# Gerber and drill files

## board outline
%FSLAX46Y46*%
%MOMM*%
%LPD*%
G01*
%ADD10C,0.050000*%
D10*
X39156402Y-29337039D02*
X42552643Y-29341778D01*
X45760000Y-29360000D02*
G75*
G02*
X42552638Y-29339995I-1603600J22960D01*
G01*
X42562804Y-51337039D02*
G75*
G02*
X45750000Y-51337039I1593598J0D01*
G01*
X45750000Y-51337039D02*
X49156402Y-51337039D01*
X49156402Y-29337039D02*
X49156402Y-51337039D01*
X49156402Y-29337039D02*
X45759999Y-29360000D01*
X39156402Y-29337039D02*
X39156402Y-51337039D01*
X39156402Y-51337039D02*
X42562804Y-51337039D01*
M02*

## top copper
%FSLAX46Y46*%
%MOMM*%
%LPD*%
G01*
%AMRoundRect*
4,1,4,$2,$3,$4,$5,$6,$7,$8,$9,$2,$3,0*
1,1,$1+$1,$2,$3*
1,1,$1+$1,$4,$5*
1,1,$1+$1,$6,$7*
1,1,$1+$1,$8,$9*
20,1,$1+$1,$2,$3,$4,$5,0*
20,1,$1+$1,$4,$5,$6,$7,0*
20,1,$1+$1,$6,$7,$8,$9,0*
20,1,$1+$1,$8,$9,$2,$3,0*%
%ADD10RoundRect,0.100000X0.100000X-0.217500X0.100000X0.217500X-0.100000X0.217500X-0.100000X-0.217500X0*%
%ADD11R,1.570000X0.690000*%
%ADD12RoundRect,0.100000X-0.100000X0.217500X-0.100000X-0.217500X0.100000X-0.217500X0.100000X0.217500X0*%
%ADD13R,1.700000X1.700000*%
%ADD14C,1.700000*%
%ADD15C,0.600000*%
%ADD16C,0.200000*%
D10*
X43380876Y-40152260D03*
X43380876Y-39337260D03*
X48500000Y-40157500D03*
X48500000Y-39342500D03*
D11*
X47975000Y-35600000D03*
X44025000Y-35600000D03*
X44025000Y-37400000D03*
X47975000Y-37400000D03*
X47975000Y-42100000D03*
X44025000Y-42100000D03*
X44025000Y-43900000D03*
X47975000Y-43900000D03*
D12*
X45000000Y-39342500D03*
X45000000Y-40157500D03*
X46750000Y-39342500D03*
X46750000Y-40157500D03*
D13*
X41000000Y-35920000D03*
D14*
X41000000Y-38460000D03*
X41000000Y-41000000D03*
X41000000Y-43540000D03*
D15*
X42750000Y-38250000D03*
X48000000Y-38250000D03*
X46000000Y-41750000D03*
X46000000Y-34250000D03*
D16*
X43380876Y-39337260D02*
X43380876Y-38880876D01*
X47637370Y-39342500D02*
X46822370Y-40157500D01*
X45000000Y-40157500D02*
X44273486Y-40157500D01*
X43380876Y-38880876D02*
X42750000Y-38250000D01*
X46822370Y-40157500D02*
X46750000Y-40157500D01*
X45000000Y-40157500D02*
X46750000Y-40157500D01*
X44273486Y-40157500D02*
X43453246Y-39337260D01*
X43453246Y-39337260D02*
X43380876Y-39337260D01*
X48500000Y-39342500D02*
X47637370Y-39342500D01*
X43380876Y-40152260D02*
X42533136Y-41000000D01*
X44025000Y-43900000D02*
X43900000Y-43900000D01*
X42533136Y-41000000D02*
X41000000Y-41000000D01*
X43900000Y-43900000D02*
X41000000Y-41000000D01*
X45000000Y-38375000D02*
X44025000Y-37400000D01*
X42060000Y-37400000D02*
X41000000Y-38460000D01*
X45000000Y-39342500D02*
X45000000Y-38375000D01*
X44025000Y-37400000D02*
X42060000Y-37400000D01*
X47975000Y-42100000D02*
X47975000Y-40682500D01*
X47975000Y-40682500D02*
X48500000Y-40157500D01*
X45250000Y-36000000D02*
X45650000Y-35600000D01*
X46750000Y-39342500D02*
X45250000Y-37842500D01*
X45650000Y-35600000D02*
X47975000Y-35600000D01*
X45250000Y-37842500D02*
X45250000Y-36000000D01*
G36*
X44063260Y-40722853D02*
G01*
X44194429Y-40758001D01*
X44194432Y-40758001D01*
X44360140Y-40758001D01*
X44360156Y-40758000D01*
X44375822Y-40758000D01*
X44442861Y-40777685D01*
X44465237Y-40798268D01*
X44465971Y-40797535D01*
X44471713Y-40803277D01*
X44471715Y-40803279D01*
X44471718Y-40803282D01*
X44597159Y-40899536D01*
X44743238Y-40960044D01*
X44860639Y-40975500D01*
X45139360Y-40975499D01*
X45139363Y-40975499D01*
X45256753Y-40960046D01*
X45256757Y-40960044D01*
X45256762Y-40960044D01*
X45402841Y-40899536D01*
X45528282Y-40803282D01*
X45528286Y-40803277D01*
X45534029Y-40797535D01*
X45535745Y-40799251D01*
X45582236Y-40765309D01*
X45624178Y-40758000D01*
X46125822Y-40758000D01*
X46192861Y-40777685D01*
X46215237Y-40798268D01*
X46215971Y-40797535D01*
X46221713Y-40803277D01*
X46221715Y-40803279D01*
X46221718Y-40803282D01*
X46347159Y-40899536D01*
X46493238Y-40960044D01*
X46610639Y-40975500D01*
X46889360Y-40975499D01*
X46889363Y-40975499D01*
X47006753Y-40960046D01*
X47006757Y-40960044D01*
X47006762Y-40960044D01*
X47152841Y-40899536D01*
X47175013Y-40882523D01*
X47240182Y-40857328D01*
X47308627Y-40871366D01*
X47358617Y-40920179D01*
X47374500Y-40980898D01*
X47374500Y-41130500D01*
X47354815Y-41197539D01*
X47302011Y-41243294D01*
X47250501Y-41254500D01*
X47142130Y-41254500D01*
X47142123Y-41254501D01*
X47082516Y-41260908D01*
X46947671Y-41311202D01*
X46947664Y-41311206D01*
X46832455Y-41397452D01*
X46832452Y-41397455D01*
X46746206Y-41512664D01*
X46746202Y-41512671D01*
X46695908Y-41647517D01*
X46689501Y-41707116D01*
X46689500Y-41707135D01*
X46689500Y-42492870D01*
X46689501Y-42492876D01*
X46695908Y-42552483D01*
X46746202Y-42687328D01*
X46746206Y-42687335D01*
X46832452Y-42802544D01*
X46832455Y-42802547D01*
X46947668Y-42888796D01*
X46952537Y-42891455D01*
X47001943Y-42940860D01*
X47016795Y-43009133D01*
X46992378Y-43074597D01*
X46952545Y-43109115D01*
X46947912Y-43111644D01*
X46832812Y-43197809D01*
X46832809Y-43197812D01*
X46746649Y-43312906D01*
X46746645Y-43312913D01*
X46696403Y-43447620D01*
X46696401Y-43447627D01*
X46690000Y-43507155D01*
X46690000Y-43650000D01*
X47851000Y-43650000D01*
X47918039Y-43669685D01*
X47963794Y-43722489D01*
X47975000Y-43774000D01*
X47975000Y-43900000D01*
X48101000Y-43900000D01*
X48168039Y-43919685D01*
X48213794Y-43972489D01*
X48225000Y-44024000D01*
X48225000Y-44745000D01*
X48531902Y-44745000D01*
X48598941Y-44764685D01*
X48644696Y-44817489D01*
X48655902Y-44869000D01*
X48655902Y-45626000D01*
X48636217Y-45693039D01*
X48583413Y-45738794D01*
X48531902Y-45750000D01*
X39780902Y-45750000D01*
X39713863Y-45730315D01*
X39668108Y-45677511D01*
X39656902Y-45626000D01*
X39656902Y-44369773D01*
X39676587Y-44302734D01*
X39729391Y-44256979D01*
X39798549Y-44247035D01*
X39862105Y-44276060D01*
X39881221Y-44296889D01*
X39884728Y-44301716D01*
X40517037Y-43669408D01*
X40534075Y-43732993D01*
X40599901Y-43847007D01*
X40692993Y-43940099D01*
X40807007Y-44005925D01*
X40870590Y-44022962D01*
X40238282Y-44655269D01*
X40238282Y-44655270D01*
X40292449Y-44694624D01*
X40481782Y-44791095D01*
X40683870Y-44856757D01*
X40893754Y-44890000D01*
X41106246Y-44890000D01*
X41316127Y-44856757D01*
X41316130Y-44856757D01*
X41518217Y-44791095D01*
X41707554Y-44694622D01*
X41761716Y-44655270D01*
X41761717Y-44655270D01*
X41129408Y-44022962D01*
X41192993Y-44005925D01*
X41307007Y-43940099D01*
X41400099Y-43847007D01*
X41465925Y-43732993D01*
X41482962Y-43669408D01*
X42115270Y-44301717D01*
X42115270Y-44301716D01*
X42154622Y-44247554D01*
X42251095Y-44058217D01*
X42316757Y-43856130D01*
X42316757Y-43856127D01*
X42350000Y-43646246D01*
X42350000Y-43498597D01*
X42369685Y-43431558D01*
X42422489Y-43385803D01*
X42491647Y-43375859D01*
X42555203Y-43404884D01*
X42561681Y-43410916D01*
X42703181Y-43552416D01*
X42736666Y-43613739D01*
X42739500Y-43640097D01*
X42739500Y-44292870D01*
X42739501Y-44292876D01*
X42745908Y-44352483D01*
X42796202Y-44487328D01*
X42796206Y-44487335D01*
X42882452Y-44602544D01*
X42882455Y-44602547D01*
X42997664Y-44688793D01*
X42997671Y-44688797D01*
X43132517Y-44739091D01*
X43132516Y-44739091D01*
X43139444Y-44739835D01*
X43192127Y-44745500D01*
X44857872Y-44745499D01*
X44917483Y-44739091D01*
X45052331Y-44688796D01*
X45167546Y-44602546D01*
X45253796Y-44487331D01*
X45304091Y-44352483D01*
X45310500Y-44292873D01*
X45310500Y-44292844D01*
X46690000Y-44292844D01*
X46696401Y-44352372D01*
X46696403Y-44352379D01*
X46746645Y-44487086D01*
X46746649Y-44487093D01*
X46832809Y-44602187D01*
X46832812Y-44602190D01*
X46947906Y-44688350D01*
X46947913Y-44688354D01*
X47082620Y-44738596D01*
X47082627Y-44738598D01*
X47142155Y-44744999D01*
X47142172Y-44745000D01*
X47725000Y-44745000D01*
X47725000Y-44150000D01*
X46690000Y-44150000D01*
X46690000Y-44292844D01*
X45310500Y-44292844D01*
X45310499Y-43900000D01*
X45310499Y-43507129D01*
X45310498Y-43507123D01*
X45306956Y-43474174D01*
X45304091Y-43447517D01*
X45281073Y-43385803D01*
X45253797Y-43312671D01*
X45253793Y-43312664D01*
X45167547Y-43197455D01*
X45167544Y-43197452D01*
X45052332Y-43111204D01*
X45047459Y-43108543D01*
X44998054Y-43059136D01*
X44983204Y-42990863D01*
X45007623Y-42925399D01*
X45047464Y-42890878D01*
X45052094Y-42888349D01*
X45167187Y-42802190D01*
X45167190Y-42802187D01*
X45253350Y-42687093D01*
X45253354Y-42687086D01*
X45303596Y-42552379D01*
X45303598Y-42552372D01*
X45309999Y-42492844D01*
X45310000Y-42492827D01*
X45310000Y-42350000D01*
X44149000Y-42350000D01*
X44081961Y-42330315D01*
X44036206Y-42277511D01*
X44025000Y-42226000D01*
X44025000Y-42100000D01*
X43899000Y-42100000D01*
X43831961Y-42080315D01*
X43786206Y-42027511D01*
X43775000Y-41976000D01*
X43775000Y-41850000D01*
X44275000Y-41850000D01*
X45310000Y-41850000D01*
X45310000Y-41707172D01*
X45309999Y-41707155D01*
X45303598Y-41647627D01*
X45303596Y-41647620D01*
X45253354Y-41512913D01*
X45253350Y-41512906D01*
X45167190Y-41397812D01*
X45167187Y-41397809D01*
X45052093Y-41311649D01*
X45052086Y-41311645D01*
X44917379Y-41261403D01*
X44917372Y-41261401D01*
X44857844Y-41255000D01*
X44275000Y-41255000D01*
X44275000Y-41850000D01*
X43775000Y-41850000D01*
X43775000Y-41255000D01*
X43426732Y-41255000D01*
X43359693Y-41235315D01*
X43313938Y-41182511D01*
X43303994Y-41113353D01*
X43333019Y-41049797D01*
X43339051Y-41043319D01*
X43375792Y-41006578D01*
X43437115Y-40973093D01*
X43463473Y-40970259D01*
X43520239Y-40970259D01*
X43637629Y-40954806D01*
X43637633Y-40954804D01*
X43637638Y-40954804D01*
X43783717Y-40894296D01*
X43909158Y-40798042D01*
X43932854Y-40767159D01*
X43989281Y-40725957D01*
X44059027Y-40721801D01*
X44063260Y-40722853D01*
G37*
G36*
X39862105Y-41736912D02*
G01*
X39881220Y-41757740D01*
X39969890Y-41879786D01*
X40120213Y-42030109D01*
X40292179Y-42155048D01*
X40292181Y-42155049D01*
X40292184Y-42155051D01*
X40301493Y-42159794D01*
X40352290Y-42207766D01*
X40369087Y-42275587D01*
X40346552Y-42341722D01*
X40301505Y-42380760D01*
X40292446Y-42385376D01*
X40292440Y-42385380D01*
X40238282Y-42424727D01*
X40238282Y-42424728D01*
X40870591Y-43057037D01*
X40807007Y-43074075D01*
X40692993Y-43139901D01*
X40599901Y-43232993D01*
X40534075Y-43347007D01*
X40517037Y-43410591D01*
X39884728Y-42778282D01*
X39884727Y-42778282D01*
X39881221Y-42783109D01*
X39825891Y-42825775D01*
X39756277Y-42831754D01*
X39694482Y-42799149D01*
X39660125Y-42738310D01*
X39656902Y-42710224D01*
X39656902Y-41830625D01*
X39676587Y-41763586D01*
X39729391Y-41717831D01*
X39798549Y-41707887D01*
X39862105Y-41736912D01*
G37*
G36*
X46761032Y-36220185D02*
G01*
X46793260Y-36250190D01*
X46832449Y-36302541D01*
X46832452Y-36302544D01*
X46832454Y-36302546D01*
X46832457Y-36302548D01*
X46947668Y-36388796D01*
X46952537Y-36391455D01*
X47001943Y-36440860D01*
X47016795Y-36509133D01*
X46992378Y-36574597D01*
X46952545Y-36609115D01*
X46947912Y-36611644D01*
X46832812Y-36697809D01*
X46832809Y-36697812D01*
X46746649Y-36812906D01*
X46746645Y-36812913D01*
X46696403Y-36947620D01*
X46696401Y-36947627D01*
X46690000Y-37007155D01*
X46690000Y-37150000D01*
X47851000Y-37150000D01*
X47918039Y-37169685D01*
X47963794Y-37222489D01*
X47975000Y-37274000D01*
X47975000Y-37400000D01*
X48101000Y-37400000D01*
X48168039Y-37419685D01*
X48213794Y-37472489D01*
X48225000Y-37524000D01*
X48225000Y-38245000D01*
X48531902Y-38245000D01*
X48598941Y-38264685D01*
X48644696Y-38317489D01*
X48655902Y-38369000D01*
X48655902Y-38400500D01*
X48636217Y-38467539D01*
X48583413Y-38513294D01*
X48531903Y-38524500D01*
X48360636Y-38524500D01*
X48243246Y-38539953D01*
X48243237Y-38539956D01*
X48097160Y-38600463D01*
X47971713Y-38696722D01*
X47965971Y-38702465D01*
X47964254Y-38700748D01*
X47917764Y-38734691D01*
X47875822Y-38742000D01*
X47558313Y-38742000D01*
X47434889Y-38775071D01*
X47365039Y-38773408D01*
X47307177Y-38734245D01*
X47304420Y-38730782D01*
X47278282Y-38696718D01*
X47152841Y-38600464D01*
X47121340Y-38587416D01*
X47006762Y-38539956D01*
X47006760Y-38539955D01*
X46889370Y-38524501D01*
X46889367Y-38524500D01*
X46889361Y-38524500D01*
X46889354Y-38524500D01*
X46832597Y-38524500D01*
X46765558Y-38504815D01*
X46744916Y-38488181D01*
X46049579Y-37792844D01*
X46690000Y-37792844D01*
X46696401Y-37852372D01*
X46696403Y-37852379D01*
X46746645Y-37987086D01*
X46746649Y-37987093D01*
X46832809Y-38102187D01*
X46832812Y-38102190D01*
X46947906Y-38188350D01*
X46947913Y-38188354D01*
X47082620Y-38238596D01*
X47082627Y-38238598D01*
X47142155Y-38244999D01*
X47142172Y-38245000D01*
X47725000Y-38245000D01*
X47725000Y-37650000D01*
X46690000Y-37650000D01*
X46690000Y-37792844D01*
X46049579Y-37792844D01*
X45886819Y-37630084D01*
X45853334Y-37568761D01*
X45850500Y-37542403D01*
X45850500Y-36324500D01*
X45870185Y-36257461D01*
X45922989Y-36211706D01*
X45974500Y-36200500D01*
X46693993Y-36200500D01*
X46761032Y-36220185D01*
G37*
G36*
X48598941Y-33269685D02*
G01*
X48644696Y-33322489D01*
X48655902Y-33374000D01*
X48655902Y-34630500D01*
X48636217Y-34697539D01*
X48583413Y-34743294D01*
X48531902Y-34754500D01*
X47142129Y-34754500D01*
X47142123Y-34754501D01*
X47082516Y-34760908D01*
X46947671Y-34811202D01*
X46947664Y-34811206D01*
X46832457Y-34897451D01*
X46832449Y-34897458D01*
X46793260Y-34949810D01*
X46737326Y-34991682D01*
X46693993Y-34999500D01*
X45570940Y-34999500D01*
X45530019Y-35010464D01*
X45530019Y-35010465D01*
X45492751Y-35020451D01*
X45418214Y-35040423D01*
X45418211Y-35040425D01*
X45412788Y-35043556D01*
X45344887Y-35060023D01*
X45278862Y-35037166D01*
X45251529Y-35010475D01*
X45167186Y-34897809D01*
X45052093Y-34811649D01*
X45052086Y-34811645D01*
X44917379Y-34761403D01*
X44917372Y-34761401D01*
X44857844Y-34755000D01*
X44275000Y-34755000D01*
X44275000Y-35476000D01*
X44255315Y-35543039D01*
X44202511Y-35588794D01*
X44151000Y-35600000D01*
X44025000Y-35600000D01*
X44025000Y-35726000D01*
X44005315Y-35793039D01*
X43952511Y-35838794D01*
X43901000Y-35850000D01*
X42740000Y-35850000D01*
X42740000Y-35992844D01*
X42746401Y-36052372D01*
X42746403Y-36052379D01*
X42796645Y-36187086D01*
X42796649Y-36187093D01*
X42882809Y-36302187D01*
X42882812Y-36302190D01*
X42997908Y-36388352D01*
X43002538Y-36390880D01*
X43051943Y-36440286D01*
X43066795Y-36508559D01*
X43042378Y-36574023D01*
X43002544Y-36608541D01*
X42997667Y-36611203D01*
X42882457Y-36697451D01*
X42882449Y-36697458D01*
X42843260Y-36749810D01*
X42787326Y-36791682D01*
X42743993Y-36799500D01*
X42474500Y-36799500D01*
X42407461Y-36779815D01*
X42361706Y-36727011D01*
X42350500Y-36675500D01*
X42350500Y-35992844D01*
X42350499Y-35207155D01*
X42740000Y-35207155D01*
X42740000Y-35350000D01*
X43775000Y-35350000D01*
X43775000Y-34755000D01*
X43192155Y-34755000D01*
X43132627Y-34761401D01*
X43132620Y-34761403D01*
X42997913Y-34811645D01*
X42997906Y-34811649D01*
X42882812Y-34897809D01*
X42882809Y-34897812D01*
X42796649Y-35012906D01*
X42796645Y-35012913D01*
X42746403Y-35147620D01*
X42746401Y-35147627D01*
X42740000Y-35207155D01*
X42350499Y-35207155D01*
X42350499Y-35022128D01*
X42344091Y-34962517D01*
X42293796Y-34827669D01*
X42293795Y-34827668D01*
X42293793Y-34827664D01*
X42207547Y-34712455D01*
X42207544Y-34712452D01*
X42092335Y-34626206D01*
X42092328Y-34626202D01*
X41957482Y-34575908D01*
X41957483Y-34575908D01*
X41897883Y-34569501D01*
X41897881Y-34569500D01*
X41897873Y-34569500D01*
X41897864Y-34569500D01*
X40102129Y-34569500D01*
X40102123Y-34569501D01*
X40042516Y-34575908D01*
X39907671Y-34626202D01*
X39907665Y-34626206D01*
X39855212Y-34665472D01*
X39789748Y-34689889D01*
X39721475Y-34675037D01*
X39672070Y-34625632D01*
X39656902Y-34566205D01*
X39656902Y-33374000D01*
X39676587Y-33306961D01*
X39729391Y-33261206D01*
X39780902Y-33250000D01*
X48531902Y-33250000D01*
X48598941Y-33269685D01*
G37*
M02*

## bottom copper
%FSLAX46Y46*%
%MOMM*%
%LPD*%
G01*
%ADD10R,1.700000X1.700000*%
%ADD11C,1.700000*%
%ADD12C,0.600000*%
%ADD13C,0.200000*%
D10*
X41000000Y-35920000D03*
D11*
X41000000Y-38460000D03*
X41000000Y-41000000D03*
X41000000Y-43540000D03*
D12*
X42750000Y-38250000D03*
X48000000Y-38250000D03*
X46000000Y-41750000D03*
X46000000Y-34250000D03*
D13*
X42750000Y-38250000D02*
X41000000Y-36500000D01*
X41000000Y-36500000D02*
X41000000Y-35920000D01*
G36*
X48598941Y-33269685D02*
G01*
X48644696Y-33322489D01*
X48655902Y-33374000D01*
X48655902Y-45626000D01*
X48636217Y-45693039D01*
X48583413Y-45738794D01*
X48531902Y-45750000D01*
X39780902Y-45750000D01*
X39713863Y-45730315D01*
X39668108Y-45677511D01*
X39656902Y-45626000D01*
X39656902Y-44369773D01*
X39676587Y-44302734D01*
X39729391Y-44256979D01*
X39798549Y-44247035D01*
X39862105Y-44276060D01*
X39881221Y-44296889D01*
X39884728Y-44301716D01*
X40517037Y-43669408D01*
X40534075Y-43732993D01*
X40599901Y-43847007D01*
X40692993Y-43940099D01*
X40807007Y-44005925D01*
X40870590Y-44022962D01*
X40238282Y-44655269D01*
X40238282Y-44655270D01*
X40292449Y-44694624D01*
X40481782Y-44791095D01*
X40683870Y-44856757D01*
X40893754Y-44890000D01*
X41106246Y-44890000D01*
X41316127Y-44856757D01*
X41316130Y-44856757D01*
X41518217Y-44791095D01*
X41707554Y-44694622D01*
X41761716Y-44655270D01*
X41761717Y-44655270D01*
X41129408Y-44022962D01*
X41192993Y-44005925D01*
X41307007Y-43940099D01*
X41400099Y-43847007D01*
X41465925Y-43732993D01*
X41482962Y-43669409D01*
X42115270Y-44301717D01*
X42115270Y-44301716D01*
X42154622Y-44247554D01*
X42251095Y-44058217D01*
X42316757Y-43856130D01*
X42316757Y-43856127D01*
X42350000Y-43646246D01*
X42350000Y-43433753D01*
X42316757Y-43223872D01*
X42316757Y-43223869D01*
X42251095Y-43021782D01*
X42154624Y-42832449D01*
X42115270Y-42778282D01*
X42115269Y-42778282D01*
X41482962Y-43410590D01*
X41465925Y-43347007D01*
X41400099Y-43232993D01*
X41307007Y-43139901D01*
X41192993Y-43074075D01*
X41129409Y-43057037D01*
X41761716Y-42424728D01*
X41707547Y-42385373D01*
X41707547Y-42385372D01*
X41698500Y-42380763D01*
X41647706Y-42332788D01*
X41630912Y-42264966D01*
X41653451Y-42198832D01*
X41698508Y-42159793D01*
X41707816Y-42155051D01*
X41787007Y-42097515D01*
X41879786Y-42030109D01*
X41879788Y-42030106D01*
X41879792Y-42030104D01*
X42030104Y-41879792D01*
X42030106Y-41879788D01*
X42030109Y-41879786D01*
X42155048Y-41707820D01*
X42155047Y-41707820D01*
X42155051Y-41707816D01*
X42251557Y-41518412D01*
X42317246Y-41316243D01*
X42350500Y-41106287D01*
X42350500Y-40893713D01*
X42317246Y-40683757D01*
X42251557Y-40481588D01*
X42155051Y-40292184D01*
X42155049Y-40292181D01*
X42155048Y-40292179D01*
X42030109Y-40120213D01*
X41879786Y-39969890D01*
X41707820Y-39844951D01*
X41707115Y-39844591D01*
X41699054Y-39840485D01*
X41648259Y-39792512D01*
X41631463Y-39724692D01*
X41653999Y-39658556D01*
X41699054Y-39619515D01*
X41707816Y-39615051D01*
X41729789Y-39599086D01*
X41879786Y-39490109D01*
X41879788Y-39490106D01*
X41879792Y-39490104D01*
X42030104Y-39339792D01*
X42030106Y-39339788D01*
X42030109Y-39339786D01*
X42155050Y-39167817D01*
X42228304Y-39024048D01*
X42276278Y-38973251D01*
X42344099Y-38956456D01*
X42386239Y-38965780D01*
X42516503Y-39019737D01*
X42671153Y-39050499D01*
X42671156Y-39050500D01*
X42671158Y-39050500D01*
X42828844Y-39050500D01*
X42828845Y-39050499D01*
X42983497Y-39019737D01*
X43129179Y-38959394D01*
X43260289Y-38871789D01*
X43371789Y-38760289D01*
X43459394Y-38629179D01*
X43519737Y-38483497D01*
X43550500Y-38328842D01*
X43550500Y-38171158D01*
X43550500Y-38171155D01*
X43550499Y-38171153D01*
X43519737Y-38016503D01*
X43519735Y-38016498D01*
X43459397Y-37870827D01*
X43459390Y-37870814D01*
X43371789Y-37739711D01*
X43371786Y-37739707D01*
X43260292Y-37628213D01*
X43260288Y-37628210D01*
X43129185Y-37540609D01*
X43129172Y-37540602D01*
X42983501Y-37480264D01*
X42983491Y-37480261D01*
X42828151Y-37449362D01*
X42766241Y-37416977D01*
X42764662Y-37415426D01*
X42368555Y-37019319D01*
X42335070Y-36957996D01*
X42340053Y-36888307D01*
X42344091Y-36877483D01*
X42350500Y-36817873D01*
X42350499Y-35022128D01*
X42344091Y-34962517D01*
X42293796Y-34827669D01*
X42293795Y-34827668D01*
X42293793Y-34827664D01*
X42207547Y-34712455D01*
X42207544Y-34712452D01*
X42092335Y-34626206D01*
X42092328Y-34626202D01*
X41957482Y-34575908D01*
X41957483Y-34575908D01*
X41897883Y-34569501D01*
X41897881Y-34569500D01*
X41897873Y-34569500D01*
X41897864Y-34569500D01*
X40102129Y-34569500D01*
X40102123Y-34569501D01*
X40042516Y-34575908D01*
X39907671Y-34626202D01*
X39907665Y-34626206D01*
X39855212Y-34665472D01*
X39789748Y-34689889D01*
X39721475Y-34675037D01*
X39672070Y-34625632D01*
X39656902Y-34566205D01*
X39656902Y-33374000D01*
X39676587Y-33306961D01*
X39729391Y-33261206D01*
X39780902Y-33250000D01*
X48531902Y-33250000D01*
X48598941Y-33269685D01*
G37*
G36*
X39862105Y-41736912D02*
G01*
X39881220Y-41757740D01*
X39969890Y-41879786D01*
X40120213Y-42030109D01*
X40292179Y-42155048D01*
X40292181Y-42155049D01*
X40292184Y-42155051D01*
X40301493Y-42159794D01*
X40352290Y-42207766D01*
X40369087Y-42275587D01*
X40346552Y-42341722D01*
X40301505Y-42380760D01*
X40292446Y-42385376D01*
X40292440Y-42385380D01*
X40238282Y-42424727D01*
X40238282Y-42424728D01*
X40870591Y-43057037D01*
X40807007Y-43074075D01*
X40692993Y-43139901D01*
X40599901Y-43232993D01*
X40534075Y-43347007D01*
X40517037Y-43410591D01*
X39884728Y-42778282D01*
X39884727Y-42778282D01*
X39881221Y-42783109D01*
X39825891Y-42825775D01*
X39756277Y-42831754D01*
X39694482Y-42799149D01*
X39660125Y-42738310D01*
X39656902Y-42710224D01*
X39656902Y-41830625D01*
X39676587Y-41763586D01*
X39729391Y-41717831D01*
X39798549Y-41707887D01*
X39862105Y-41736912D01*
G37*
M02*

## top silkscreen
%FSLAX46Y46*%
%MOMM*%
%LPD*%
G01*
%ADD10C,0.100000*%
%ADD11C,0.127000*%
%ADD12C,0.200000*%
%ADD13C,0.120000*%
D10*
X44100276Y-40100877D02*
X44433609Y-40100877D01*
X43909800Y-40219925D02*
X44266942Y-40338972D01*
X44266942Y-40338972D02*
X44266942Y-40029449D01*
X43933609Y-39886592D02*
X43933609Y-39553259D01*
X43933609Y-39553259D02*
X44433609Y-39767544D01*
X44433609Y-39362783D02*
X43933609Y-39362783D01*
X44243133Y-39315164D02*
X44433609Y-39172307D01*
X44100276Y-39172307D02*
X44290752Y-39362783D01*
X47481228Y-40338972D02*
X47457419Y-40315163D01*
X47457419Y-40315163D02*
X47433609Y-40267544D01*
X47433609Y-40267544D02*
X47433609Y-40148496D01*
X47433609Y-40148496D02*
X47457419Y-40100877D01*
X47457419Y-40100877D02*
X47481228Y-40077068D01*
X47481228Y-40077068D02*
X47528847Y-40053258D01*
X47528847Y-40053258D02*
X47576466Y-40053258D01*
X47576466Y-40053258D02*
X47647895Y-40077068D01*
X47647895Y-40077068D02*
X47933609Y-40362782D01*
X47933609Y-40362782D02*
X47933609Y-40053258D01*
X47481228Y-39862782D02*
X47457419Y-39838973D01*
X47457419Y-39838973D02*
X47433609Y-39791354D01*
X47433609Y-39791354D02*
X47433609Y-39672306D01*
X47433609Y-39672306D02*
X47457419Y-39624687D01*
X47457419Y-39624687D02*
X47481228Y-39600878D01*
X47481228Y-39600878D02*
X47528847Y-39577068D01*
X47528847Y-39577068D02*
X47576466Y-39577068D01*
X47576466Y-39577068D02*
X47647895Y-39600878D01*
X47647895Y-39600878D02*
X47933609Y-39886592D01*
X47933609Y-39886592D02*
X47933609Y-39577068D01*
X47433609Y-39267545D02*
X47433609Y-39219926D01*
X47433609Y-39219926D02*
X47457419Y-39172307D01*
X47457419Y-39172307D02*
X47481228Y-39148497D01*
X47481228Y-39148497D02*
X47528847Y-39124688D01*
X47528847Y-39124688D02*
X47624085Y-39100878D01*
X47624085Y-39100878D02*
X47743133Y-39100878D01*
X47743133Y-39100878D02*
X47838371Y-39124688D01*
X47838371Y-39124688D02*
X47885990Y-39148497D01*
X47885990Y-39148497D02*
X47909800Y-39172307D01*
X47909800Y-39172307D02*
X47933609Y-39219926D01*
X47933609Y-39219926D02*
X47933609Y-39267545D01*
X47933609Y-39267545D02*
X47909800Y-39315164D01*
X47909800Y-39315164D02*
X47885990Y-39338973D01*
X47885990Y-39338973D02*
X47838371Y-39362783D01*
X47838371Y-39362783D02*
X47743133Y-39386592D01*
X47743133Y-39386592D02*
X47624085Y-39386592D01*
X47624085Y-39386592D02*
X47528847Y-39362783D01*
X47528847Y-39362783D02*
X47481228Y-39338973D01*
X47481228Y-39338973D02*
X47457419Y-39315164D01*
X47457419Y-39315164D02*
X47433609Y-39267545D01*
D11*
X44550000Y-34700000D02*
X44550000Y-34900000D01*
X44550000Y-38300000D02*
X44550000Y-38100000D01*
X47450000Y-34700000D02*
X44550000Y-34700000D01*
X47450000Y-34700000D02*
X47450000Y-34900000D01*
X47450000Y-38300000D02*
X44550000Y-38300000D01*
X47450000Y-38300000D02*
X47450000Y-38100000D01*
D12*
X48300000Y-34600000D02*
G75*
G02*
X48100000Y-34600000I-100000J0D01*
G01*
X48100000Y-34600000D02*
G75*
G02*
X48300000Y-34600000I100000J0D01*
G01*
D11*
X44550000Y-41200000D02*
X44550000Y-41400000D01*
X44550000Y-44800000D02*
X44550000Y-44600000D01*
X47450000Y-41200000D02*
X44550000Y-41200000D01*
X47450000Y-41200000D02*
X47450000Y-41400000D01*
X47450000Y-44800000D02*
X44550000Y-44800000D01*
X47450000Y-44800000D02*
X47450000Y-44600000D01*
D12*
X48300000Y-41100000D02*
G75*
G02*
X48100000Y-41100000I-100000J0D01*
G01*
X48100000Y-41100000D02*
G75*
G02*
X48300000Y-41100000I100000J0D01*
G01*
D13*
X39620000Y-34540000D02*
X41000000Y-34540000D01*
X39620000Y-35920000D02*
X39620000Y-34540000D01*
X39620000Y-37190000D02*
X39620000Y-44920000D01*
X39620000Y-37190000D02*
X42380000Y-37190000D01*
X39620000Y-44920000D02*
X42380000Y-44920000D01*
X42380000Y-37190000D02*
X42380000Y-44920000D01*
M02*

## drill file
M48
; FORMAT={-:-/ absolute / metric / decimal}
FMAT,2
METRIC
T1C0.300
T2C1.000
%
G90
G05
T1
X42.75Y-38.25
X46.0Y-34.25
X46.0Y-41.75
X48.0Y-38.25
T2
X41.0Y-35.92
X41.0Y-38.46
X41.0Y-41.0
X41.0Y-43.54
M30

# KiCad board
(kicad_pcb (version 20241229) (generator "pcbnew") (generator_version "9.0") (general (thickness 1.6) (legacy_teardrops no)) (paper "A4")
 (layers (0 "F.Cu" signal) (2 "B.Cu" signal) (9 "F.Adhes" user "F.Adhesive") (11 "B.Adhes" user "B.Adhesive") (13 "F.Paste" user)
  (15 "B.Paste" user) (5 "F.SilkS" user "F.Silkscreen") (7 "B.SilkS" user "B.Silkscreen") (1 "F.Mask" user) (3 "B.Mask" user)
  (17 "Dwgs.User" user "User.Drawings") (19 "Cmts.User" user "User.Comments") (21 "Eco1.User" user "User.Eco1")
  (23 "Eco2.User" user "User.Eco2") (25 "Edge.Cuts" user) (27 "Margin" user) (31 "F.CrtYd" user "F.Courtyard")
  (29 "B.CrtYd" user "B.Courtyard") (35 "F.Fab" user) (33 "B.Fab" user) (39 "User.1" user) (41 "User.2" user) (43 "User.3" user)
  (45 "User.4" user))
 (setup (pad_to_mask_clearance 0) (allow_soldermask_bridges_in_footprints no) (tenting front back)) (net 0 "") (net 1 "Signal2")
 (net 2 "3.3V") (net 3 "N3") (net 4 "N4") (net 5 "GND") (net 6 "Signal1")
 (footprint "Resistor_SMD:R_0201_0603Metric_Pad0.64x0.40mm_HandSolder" (layer "F.Cu") (at 43.380876 39.74476 90)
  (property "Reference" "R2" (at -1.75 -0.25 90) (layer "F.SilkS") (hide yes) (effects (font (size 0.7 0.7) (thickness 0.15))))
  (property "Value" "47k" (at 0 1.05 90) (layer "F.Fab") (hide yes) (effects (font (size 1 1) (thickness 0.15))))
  (pad "" smd roundrect (at -0.4325 0 90) (size 0.458 0.36) (layers "F.Paste") (roundrect_rratio 0.25))
  (pad "" smd roundrect (at 0.4325 0 90) (size 0.458 0.36) (layers "F.Paste") (roundrect_rratio 0.25))
  (pad "1" smd roundrect (at -0.4075 0 90) (size 0.635 0.4) (layers "F.Cu" "F.Mask") (roundrect_rratio 0.25) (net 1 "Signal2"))
  (pad "2" smd roundrect (at 0.4075 0 90) (size 0.635 0.4) (layers "F.Cu" "F.Mask") (roundrect_rratio 0.25) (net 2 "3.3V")))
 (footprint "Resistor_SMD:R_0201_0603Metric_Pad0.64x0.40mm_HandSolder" (layer "F.Cu") (at 48.5 39.75 90)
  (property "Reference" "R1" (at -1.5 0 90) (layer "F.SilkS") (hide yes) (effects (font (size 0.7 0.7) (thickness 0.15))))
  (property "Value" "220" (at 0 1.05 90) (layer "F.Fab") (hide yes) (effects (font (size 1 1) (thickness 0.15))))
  (pad "" smd roundrect (at -0.4325 0 90) (size 0.458 0.36) (layers "F.Paste") (roundrect_rratio 0.25))
  (pad "" smd roundrect (at 0.4325 0 90) (size 0.458 0.36) (layers "F.Paste") (roundrect_rratio 0.25))
  (pad "1" smd roundrect (at -0.4075 0 90) (size 0.635 0.4) (layers "F.Cu" "F.Mask") (roundrect_rratio 0.25) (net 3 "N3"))
  (pad "2" smd roundrect (at 0.4075 0 90) (size 0.635 0.4) (layers "F.Cu" "F.Mask") (roundrect_rratio 0.25) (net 2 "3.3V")))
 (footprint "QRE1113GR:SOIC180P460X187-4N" (layer "F.Cu") (at 46 36.5 -90)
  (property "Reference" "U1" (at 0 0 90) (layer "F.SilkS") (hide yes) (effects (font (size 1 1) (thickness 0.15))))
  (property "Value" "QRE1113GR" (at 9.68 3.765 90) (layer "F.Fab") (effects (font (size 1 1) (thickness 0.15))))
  (fp_line (start -1.8 1.45) (end -1.6 1.45) (stroke (width 0.127) (type solid)) (layer "F.SilkS"))
  (fp_line (start 1.8 1.45) (end 1.6 1.45) (stroke (width 0.127) (type solid)) (layer "F.SilkS"))
  (fp_line (start -1.8 -1.45) (end -1.8 1.45) (stroke (width 0.127) (type solid)) (layer "F.SilkS"))
  (fp_line (start -1.8 -1.45) (end -1.6 -1.45) (stroke (width 0.127) (type solid)) (layer "F.SilkS"))
  (fp_line (start 1.8 -1.45) (end 1.8 1.45) (stroke (width 0.127) (type solid)) (layer "F.SilkS"))
  (fp_line (start 1.8 -1.45) (end 1.6 -1.45) (stroke (width 0.127) (type solid)) (layer "F.SilkS"))
  (fp_circle (center -1.9 -2.2) (end -1.8 -2.2) (stroke (width 0.2) (type solid)) (fill no) (layer "F.SilkS"))
  (pad "1" smd rect (at -0.9 -1.975 270) (size 0.69 1.57) (layers "F.Cu" "F.Mask" "F.Paste") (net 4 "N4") (solder_mask_margin 0.102))
  (pad "2" smd rect (at -0.9 1.975 270) (size 0.69 1.57) (layers "F.Cu" "F.Mask" "F.Paste") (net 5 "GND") (solder_mask_margin 0.102))
  (pad "3" smd rect (at 0.9 1.975 270) (size 0.69 1.57) (layers "F.Cu" "F.Mask" "F.Paste") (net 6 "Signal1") (solder_mask_margin 0.102))
  (pad "4" smd rect (at 0.9 -1.975 270) (size 0.69 1.57) (layers "F.Cu" "F.Mask" "F.Paste") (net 5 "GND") (solder_mask_margin 0.102)))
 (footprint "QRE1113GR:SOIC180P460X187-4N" (layer "F.Cu") (at 46 43 -90)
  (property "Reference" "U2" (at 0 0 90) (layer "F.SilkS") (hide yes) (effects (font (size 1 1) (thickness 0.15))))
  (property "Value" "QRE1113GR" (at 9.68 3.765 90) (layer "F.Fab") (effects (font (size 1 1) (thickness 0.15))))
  (fp_line (start -1.8 1.45) (end -1.6 1.45) (stroke (width 0.127) (type solid)) (layer "F.SilkS"))
  (fp_line (start 1.8 1.45) (end 1.6 1.45) (stroke (width 0.127) (type solid)) (layer "F.SilkS"))
  (fp_line (start -1.8 -1.45) (end -1.8 1.45) (stroke (width 0.127) (type solid)) (layer "F.SilkS"))
  (fp_line (start -1.8 -1.45) (end -1.6 -1.45) (stroke (width 0.127) (type solid)) (layer "F.SilkS"))
  (fp_line (start 1.8 -1.45) (end 1.8 1.45) (stroke (width 0.127) (type solid)) (layer "F.SilkS"))
  (fp_line (start 1.8 -1.45) (end 1.6 -1.45) (stroke (width 0.127) (type solid)) (layer "F.SilkS"))
  (fp_circle (center -1.9 -2.2) (end -1.8 -2.2) (stroke (width 0.2) (type solid)) (fill no) (layer "F.SilkS"))
  (pad "1" smd rect (at -0.9 -1.975 270) (size 0.69 1.57) (layers "F.Cu" "F.Mask" "F.Paste") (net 3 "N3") (solder_mask_margin 0.102))
  (pad "2" smd rect (at -0.9 1.975 270) (size 0.69 1.57) (layers "F.Cu" "F.Mask" "F.Paste") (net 5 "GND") (solder_mask_margin 0.102))
  (pad "3" smd rect (at 0.9 1.975 270) (size 0.69 1.57) (layers "F.Cu" "F.Mask" "F.Paste") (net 1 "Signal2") (solder_mask_margin 0.102))
  (pad "4" smd rect (at 0.9 -1.975 270) (size 0.69 1.57) (layers "F.Cu" "F.Mask" "F.Paste") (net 5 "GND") (solder_mask_margin 0.102)))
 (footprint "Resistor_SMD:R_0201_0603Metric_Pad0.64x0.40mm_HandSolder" (layer "F.Cu") (at 45 39.75 -90)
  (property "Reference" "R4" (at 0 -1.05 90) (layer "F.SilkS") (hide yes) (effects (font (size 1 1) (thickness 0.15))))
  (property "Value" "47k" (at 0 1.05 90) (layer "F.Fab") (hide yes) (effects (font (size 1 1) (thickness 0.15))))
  (pad "" smd roundrect (at -0.4325 0 270) (size 0.458 0.36) (layers "F.Paste") (roundrect_rratio 0.25))
  (pad "" smd roundrect (at 0.4325 0 270) (size 0.458 0.36) (layers "F.Paste") (roundrect_rratio 0.25))
  (pad "1" smd roundrect (at -0.4075 0 270) (size 0.635 0.4) (layers "F.Cu" "F.Mask") (roundrect_rratio 0.25) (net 6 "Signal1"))
  (pad "2" smd roundrect (at 0.4075 0 270) (size 0.635 0.4) (layers "F.Cu" "F.Mask") (roundrect_rratio 0.25) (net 2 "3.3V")))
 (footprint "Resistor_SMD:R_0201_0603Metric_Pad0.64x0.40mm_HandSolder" (layer "F.Cu") (at 46.75 39.75 -90)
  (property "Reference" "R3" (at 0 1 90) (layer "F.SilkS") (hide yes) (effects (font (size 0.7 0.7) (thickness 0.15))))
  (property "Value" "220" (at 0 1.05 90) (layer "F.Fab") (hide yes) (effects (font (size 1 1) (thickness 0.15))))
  (pad "" smd roundrect (at -0.4325 0 270) (size 0.458 0.36) (layers "F.Paste") (roundrect_rratio 0.25))
  (pad "" smd roundrect (at 0.4325 0 270) (size 0.458 0.36) (layers "F.Paste") (roundrect_rratio 0.25))
  (pad "1" smd roundrect (at -0.4075 0 270) (size 0.635 0.4) (layers "F.Cu" "F.Mask") (roundrect_rratio 0.25) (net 4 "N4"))
  (pad "2" smd roundrect (at 0.4075 0 270) (size 0.635 0.4) (layers "F.Cu" "F.Mask") (roundrect_rratio 0.25) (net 2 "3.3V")))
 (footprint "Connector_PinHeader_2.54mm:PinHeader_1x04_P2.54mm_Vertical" (layer "F.Cu") (at 41 35.92)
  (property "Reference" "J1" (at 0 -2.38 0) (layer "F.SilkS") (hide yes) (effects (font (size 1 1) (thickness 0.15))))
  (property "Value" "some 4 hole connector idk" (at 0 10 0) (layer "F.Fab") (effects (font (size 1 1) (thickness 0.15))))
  (fp_line (start -1.38 -1.38) (end 0 -1.38) (stroke (width 0.12) (type solid)) (layer "F.SilkS"))
  (fp_line (start -1.38 0) (end -1.38 -1.38) (stroke (width 0.12) (type solid)) (layer "F.SilkS"))
  (fp_line (start -1.38 1.27) (end -1.38 9) (stroke (width 0.12) (type solid)) (layer "F.SilkS"))
  (fp_line (start -1.38 1.27) (end 1.38 1.27) (stroke (width 0.12) (type solid)) (layer "F.SilkS"))
  (fp_line (start -1.38 9) (end 1.38 9) (stroke (width 0.12) (type solid)) (layer "F.SilkS"))
  (fp_line (start 1.38 1.27) (end 1.38 9) (stroke (width 0.12) (type solid)) (layer "F.SilkS"))
  (pad "1" thru_hole rect (at 0 0) (size 1.7 1.7) (drill 1) (layers "*.Cu" "*.Mask") (remove_unused_layers no) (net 2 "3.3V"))
  (pad "2" thru_hole circle (at 0 2.54) (size 1.7 1.7) (drill 1) (layers "*.Cu" "*.Mask") (remove_unused_layers no) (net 6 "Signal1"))
  (pad "3" thru_hole circle (at 0 5.08) (size 1.7 1.7) (drill 1) (layers "*.Cu" "*.Mask") (remove_unused_layers no) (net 1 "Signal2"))
  (pad "4" thru_hole circle (at 0 7.62) (size 1.7 1.7) (drill 1) (layers "*.Cu" "*.Mask") (remove_unused_layers no) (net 5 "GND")))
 (gr_line (start 39.156402 29.337039) (end 42.552643 29.341778) (stroke (width 0.05) (type default)) (layer "Edge.Cuts"))
 (gr_arc (start 45.76 29.36) (mid 44.146399 30.94077) (end 42.552643 29.339995) (stroke (width 0.05) (type default)) (layer "Edge.Cuts"))
 (gr_arc (start 42.562804 51.337039) (mid 44.156402 49.743441) (end 45.75 51.337039) (stroke (width 0.05) (type solid)) (layer "Edge.Cuts"))
 (gr_line (start 45.75 51.337039) (end 49.156402 51.337039) (stroke (width 0.05) (type default)) (layer "Edge.Cuts"))
 (gr_line (start 49.156402 29.337039) (end 49.156402 51.337039) (stroke (width 0.05) (type default)) (layer "Edge.Cuts"))
 (gr_line (start 49.156402 29.337039) (end 45.759999 29.36) (stroke (width 0.05) (type default)) (layer "Edge.Cuts"))
 (gr_line (start 39.156402 29.337039) (end 39.156402 51.337039) (stroke (width 0.05) (type default)) (layer "Edge.Cuts"))
 (gr_line (start 39.156402 51.337039) (end 42.562804 51.337039) (stroke (width 0.05) (type default)) (layer "Edge.Cuts"))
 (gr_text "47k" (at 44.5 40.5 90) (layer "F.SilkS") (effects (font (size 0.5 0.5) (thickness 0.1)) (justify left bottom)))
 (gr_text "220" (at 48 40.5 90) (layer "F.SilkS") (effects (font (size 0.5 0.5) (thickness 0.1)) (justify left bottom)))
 (segment (start 43.380876 39.33726) (end 43.380876 38.880876) (width 0.2) (layer "F.Cu") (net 2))
 (segment (start 47.63737 39.3425) (end 46.82237 40.1575) (width 0.2) (layer "F.Cu") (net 2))
 (segment (start 45 40.1575) (end 44.273486 40.1575) (width 0.2) (layer "F.Cu") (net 2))
 (segment (start 43.380876 38.880876) (end 42.75 38.25) (width 0.2) (layer "F.Cu") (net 2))
 (segment (start 46.82237 40.1575) (end 46.75 40.1575) (width 0.2) (layer "F.Cu") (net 2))
 (segment (start 45 40.1575) (end 46.75 40.1575) (width 0.2) (layer "F.Cu") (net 2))
 (segment (start 44.273486 40.1575) (end 43.453246 39.33726) (width 0.2) (layer "F.Cu") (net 2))
 (segment (start 43.453246 39.33726) (end 43.380876 39.33726) (width 0.2) (layer "F.Cu") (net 2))
 (segment (start 48.5 39.3425) (end 47.63737 39.3425) (width 0.2) (layer "F.Cu") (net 2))
 (via (at 42.75 38.25) (size 0.6) (drill 0.3) (layers "F.Cu" "B.Cu") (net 2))
 (segment (start 42.75 38.25) (end 41 36.5) (width 0.2) (layer "B.Cu") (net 2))
 (segment (start 41 36.5) (end 41 35.92) (width 0.2) (layer "B.Cu") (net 2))
 (via (at 48 38.25) (size 0.6) (drill 0.3) (layers "F.Cu" "B.Cu") (free yes) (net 5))
 (via (at 46 41.75) (size 0.6) (drill 0.3) (layers "F.Cu" "B.Cu") (free yes) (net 5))
 (via (at 46 34.25) (size 0.6) (drill 0.3) (layers "F.Cu" "B.Cu") (free yes) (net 5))
 (segment (start 43.380876 40.15226) (end 42.533136 41) (width 0.2) (layer "F.Cu") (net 1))
 (segment (start 44.025 43.9) (end 43.9 43.9) (width 0.2) (layer "F.Cu") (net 1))
 (segment (start 42.533136 41) (end 41 41) (width 0.2) (layer "F.Cu") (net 1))
 (segment (start 43.9 43.9) (end 41 41) (width 0.2) (layer "F.Cu") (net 1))
 (segment (start 45 38.375) (end 44.025 37.4) (width 0.2) (layer "F.Cu") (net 6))
 (segment (start 42.06 37.4) (end 41 38.46) (width 0.2) (layer "F.Cu") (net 6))
 (segment (start 45 39.3425) (end 45 38.375) (width 0.2) (layer "F.Cu") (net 6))
 (segment (start 44.025 37.4) (end 42.06 37.4) (width 0.2) (layer "F.Cu") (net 6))
 (segment (start 47.975 42.1) (end 47.975 40.6825) (width 0.2) (layer "F.Cu") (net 3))
 (segment (start 47.975 40.6825) (end 48.5 40.1575) (width 0.2) (layer "F.Cu") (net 3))
 (segment (start 45.25 36) (end 45.65 35.6) (width 0.2) (layer "F.Cu") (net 4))
 (segment (start 46.75 39.3425) (end 45.25 37.8425) (width 0.2) (layer "F.Cu") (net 4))
 (segment (start 45.65 35.6) (end 47.975 35.6) (width 0.2) (layer "F.Cu") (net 4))
 (segment (start 45.25 37.8425) (end 45.25 36) (width 0.2) (layer "F.Cu") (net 4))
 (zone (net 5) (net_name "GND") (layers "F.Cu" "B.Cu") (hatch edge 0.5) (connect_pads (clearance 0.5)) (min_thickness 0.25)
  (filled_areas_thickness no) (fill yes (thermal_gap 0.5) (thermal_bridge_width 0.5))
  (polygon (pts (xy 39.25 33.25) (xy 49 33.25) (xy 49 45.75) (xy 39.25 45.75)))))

